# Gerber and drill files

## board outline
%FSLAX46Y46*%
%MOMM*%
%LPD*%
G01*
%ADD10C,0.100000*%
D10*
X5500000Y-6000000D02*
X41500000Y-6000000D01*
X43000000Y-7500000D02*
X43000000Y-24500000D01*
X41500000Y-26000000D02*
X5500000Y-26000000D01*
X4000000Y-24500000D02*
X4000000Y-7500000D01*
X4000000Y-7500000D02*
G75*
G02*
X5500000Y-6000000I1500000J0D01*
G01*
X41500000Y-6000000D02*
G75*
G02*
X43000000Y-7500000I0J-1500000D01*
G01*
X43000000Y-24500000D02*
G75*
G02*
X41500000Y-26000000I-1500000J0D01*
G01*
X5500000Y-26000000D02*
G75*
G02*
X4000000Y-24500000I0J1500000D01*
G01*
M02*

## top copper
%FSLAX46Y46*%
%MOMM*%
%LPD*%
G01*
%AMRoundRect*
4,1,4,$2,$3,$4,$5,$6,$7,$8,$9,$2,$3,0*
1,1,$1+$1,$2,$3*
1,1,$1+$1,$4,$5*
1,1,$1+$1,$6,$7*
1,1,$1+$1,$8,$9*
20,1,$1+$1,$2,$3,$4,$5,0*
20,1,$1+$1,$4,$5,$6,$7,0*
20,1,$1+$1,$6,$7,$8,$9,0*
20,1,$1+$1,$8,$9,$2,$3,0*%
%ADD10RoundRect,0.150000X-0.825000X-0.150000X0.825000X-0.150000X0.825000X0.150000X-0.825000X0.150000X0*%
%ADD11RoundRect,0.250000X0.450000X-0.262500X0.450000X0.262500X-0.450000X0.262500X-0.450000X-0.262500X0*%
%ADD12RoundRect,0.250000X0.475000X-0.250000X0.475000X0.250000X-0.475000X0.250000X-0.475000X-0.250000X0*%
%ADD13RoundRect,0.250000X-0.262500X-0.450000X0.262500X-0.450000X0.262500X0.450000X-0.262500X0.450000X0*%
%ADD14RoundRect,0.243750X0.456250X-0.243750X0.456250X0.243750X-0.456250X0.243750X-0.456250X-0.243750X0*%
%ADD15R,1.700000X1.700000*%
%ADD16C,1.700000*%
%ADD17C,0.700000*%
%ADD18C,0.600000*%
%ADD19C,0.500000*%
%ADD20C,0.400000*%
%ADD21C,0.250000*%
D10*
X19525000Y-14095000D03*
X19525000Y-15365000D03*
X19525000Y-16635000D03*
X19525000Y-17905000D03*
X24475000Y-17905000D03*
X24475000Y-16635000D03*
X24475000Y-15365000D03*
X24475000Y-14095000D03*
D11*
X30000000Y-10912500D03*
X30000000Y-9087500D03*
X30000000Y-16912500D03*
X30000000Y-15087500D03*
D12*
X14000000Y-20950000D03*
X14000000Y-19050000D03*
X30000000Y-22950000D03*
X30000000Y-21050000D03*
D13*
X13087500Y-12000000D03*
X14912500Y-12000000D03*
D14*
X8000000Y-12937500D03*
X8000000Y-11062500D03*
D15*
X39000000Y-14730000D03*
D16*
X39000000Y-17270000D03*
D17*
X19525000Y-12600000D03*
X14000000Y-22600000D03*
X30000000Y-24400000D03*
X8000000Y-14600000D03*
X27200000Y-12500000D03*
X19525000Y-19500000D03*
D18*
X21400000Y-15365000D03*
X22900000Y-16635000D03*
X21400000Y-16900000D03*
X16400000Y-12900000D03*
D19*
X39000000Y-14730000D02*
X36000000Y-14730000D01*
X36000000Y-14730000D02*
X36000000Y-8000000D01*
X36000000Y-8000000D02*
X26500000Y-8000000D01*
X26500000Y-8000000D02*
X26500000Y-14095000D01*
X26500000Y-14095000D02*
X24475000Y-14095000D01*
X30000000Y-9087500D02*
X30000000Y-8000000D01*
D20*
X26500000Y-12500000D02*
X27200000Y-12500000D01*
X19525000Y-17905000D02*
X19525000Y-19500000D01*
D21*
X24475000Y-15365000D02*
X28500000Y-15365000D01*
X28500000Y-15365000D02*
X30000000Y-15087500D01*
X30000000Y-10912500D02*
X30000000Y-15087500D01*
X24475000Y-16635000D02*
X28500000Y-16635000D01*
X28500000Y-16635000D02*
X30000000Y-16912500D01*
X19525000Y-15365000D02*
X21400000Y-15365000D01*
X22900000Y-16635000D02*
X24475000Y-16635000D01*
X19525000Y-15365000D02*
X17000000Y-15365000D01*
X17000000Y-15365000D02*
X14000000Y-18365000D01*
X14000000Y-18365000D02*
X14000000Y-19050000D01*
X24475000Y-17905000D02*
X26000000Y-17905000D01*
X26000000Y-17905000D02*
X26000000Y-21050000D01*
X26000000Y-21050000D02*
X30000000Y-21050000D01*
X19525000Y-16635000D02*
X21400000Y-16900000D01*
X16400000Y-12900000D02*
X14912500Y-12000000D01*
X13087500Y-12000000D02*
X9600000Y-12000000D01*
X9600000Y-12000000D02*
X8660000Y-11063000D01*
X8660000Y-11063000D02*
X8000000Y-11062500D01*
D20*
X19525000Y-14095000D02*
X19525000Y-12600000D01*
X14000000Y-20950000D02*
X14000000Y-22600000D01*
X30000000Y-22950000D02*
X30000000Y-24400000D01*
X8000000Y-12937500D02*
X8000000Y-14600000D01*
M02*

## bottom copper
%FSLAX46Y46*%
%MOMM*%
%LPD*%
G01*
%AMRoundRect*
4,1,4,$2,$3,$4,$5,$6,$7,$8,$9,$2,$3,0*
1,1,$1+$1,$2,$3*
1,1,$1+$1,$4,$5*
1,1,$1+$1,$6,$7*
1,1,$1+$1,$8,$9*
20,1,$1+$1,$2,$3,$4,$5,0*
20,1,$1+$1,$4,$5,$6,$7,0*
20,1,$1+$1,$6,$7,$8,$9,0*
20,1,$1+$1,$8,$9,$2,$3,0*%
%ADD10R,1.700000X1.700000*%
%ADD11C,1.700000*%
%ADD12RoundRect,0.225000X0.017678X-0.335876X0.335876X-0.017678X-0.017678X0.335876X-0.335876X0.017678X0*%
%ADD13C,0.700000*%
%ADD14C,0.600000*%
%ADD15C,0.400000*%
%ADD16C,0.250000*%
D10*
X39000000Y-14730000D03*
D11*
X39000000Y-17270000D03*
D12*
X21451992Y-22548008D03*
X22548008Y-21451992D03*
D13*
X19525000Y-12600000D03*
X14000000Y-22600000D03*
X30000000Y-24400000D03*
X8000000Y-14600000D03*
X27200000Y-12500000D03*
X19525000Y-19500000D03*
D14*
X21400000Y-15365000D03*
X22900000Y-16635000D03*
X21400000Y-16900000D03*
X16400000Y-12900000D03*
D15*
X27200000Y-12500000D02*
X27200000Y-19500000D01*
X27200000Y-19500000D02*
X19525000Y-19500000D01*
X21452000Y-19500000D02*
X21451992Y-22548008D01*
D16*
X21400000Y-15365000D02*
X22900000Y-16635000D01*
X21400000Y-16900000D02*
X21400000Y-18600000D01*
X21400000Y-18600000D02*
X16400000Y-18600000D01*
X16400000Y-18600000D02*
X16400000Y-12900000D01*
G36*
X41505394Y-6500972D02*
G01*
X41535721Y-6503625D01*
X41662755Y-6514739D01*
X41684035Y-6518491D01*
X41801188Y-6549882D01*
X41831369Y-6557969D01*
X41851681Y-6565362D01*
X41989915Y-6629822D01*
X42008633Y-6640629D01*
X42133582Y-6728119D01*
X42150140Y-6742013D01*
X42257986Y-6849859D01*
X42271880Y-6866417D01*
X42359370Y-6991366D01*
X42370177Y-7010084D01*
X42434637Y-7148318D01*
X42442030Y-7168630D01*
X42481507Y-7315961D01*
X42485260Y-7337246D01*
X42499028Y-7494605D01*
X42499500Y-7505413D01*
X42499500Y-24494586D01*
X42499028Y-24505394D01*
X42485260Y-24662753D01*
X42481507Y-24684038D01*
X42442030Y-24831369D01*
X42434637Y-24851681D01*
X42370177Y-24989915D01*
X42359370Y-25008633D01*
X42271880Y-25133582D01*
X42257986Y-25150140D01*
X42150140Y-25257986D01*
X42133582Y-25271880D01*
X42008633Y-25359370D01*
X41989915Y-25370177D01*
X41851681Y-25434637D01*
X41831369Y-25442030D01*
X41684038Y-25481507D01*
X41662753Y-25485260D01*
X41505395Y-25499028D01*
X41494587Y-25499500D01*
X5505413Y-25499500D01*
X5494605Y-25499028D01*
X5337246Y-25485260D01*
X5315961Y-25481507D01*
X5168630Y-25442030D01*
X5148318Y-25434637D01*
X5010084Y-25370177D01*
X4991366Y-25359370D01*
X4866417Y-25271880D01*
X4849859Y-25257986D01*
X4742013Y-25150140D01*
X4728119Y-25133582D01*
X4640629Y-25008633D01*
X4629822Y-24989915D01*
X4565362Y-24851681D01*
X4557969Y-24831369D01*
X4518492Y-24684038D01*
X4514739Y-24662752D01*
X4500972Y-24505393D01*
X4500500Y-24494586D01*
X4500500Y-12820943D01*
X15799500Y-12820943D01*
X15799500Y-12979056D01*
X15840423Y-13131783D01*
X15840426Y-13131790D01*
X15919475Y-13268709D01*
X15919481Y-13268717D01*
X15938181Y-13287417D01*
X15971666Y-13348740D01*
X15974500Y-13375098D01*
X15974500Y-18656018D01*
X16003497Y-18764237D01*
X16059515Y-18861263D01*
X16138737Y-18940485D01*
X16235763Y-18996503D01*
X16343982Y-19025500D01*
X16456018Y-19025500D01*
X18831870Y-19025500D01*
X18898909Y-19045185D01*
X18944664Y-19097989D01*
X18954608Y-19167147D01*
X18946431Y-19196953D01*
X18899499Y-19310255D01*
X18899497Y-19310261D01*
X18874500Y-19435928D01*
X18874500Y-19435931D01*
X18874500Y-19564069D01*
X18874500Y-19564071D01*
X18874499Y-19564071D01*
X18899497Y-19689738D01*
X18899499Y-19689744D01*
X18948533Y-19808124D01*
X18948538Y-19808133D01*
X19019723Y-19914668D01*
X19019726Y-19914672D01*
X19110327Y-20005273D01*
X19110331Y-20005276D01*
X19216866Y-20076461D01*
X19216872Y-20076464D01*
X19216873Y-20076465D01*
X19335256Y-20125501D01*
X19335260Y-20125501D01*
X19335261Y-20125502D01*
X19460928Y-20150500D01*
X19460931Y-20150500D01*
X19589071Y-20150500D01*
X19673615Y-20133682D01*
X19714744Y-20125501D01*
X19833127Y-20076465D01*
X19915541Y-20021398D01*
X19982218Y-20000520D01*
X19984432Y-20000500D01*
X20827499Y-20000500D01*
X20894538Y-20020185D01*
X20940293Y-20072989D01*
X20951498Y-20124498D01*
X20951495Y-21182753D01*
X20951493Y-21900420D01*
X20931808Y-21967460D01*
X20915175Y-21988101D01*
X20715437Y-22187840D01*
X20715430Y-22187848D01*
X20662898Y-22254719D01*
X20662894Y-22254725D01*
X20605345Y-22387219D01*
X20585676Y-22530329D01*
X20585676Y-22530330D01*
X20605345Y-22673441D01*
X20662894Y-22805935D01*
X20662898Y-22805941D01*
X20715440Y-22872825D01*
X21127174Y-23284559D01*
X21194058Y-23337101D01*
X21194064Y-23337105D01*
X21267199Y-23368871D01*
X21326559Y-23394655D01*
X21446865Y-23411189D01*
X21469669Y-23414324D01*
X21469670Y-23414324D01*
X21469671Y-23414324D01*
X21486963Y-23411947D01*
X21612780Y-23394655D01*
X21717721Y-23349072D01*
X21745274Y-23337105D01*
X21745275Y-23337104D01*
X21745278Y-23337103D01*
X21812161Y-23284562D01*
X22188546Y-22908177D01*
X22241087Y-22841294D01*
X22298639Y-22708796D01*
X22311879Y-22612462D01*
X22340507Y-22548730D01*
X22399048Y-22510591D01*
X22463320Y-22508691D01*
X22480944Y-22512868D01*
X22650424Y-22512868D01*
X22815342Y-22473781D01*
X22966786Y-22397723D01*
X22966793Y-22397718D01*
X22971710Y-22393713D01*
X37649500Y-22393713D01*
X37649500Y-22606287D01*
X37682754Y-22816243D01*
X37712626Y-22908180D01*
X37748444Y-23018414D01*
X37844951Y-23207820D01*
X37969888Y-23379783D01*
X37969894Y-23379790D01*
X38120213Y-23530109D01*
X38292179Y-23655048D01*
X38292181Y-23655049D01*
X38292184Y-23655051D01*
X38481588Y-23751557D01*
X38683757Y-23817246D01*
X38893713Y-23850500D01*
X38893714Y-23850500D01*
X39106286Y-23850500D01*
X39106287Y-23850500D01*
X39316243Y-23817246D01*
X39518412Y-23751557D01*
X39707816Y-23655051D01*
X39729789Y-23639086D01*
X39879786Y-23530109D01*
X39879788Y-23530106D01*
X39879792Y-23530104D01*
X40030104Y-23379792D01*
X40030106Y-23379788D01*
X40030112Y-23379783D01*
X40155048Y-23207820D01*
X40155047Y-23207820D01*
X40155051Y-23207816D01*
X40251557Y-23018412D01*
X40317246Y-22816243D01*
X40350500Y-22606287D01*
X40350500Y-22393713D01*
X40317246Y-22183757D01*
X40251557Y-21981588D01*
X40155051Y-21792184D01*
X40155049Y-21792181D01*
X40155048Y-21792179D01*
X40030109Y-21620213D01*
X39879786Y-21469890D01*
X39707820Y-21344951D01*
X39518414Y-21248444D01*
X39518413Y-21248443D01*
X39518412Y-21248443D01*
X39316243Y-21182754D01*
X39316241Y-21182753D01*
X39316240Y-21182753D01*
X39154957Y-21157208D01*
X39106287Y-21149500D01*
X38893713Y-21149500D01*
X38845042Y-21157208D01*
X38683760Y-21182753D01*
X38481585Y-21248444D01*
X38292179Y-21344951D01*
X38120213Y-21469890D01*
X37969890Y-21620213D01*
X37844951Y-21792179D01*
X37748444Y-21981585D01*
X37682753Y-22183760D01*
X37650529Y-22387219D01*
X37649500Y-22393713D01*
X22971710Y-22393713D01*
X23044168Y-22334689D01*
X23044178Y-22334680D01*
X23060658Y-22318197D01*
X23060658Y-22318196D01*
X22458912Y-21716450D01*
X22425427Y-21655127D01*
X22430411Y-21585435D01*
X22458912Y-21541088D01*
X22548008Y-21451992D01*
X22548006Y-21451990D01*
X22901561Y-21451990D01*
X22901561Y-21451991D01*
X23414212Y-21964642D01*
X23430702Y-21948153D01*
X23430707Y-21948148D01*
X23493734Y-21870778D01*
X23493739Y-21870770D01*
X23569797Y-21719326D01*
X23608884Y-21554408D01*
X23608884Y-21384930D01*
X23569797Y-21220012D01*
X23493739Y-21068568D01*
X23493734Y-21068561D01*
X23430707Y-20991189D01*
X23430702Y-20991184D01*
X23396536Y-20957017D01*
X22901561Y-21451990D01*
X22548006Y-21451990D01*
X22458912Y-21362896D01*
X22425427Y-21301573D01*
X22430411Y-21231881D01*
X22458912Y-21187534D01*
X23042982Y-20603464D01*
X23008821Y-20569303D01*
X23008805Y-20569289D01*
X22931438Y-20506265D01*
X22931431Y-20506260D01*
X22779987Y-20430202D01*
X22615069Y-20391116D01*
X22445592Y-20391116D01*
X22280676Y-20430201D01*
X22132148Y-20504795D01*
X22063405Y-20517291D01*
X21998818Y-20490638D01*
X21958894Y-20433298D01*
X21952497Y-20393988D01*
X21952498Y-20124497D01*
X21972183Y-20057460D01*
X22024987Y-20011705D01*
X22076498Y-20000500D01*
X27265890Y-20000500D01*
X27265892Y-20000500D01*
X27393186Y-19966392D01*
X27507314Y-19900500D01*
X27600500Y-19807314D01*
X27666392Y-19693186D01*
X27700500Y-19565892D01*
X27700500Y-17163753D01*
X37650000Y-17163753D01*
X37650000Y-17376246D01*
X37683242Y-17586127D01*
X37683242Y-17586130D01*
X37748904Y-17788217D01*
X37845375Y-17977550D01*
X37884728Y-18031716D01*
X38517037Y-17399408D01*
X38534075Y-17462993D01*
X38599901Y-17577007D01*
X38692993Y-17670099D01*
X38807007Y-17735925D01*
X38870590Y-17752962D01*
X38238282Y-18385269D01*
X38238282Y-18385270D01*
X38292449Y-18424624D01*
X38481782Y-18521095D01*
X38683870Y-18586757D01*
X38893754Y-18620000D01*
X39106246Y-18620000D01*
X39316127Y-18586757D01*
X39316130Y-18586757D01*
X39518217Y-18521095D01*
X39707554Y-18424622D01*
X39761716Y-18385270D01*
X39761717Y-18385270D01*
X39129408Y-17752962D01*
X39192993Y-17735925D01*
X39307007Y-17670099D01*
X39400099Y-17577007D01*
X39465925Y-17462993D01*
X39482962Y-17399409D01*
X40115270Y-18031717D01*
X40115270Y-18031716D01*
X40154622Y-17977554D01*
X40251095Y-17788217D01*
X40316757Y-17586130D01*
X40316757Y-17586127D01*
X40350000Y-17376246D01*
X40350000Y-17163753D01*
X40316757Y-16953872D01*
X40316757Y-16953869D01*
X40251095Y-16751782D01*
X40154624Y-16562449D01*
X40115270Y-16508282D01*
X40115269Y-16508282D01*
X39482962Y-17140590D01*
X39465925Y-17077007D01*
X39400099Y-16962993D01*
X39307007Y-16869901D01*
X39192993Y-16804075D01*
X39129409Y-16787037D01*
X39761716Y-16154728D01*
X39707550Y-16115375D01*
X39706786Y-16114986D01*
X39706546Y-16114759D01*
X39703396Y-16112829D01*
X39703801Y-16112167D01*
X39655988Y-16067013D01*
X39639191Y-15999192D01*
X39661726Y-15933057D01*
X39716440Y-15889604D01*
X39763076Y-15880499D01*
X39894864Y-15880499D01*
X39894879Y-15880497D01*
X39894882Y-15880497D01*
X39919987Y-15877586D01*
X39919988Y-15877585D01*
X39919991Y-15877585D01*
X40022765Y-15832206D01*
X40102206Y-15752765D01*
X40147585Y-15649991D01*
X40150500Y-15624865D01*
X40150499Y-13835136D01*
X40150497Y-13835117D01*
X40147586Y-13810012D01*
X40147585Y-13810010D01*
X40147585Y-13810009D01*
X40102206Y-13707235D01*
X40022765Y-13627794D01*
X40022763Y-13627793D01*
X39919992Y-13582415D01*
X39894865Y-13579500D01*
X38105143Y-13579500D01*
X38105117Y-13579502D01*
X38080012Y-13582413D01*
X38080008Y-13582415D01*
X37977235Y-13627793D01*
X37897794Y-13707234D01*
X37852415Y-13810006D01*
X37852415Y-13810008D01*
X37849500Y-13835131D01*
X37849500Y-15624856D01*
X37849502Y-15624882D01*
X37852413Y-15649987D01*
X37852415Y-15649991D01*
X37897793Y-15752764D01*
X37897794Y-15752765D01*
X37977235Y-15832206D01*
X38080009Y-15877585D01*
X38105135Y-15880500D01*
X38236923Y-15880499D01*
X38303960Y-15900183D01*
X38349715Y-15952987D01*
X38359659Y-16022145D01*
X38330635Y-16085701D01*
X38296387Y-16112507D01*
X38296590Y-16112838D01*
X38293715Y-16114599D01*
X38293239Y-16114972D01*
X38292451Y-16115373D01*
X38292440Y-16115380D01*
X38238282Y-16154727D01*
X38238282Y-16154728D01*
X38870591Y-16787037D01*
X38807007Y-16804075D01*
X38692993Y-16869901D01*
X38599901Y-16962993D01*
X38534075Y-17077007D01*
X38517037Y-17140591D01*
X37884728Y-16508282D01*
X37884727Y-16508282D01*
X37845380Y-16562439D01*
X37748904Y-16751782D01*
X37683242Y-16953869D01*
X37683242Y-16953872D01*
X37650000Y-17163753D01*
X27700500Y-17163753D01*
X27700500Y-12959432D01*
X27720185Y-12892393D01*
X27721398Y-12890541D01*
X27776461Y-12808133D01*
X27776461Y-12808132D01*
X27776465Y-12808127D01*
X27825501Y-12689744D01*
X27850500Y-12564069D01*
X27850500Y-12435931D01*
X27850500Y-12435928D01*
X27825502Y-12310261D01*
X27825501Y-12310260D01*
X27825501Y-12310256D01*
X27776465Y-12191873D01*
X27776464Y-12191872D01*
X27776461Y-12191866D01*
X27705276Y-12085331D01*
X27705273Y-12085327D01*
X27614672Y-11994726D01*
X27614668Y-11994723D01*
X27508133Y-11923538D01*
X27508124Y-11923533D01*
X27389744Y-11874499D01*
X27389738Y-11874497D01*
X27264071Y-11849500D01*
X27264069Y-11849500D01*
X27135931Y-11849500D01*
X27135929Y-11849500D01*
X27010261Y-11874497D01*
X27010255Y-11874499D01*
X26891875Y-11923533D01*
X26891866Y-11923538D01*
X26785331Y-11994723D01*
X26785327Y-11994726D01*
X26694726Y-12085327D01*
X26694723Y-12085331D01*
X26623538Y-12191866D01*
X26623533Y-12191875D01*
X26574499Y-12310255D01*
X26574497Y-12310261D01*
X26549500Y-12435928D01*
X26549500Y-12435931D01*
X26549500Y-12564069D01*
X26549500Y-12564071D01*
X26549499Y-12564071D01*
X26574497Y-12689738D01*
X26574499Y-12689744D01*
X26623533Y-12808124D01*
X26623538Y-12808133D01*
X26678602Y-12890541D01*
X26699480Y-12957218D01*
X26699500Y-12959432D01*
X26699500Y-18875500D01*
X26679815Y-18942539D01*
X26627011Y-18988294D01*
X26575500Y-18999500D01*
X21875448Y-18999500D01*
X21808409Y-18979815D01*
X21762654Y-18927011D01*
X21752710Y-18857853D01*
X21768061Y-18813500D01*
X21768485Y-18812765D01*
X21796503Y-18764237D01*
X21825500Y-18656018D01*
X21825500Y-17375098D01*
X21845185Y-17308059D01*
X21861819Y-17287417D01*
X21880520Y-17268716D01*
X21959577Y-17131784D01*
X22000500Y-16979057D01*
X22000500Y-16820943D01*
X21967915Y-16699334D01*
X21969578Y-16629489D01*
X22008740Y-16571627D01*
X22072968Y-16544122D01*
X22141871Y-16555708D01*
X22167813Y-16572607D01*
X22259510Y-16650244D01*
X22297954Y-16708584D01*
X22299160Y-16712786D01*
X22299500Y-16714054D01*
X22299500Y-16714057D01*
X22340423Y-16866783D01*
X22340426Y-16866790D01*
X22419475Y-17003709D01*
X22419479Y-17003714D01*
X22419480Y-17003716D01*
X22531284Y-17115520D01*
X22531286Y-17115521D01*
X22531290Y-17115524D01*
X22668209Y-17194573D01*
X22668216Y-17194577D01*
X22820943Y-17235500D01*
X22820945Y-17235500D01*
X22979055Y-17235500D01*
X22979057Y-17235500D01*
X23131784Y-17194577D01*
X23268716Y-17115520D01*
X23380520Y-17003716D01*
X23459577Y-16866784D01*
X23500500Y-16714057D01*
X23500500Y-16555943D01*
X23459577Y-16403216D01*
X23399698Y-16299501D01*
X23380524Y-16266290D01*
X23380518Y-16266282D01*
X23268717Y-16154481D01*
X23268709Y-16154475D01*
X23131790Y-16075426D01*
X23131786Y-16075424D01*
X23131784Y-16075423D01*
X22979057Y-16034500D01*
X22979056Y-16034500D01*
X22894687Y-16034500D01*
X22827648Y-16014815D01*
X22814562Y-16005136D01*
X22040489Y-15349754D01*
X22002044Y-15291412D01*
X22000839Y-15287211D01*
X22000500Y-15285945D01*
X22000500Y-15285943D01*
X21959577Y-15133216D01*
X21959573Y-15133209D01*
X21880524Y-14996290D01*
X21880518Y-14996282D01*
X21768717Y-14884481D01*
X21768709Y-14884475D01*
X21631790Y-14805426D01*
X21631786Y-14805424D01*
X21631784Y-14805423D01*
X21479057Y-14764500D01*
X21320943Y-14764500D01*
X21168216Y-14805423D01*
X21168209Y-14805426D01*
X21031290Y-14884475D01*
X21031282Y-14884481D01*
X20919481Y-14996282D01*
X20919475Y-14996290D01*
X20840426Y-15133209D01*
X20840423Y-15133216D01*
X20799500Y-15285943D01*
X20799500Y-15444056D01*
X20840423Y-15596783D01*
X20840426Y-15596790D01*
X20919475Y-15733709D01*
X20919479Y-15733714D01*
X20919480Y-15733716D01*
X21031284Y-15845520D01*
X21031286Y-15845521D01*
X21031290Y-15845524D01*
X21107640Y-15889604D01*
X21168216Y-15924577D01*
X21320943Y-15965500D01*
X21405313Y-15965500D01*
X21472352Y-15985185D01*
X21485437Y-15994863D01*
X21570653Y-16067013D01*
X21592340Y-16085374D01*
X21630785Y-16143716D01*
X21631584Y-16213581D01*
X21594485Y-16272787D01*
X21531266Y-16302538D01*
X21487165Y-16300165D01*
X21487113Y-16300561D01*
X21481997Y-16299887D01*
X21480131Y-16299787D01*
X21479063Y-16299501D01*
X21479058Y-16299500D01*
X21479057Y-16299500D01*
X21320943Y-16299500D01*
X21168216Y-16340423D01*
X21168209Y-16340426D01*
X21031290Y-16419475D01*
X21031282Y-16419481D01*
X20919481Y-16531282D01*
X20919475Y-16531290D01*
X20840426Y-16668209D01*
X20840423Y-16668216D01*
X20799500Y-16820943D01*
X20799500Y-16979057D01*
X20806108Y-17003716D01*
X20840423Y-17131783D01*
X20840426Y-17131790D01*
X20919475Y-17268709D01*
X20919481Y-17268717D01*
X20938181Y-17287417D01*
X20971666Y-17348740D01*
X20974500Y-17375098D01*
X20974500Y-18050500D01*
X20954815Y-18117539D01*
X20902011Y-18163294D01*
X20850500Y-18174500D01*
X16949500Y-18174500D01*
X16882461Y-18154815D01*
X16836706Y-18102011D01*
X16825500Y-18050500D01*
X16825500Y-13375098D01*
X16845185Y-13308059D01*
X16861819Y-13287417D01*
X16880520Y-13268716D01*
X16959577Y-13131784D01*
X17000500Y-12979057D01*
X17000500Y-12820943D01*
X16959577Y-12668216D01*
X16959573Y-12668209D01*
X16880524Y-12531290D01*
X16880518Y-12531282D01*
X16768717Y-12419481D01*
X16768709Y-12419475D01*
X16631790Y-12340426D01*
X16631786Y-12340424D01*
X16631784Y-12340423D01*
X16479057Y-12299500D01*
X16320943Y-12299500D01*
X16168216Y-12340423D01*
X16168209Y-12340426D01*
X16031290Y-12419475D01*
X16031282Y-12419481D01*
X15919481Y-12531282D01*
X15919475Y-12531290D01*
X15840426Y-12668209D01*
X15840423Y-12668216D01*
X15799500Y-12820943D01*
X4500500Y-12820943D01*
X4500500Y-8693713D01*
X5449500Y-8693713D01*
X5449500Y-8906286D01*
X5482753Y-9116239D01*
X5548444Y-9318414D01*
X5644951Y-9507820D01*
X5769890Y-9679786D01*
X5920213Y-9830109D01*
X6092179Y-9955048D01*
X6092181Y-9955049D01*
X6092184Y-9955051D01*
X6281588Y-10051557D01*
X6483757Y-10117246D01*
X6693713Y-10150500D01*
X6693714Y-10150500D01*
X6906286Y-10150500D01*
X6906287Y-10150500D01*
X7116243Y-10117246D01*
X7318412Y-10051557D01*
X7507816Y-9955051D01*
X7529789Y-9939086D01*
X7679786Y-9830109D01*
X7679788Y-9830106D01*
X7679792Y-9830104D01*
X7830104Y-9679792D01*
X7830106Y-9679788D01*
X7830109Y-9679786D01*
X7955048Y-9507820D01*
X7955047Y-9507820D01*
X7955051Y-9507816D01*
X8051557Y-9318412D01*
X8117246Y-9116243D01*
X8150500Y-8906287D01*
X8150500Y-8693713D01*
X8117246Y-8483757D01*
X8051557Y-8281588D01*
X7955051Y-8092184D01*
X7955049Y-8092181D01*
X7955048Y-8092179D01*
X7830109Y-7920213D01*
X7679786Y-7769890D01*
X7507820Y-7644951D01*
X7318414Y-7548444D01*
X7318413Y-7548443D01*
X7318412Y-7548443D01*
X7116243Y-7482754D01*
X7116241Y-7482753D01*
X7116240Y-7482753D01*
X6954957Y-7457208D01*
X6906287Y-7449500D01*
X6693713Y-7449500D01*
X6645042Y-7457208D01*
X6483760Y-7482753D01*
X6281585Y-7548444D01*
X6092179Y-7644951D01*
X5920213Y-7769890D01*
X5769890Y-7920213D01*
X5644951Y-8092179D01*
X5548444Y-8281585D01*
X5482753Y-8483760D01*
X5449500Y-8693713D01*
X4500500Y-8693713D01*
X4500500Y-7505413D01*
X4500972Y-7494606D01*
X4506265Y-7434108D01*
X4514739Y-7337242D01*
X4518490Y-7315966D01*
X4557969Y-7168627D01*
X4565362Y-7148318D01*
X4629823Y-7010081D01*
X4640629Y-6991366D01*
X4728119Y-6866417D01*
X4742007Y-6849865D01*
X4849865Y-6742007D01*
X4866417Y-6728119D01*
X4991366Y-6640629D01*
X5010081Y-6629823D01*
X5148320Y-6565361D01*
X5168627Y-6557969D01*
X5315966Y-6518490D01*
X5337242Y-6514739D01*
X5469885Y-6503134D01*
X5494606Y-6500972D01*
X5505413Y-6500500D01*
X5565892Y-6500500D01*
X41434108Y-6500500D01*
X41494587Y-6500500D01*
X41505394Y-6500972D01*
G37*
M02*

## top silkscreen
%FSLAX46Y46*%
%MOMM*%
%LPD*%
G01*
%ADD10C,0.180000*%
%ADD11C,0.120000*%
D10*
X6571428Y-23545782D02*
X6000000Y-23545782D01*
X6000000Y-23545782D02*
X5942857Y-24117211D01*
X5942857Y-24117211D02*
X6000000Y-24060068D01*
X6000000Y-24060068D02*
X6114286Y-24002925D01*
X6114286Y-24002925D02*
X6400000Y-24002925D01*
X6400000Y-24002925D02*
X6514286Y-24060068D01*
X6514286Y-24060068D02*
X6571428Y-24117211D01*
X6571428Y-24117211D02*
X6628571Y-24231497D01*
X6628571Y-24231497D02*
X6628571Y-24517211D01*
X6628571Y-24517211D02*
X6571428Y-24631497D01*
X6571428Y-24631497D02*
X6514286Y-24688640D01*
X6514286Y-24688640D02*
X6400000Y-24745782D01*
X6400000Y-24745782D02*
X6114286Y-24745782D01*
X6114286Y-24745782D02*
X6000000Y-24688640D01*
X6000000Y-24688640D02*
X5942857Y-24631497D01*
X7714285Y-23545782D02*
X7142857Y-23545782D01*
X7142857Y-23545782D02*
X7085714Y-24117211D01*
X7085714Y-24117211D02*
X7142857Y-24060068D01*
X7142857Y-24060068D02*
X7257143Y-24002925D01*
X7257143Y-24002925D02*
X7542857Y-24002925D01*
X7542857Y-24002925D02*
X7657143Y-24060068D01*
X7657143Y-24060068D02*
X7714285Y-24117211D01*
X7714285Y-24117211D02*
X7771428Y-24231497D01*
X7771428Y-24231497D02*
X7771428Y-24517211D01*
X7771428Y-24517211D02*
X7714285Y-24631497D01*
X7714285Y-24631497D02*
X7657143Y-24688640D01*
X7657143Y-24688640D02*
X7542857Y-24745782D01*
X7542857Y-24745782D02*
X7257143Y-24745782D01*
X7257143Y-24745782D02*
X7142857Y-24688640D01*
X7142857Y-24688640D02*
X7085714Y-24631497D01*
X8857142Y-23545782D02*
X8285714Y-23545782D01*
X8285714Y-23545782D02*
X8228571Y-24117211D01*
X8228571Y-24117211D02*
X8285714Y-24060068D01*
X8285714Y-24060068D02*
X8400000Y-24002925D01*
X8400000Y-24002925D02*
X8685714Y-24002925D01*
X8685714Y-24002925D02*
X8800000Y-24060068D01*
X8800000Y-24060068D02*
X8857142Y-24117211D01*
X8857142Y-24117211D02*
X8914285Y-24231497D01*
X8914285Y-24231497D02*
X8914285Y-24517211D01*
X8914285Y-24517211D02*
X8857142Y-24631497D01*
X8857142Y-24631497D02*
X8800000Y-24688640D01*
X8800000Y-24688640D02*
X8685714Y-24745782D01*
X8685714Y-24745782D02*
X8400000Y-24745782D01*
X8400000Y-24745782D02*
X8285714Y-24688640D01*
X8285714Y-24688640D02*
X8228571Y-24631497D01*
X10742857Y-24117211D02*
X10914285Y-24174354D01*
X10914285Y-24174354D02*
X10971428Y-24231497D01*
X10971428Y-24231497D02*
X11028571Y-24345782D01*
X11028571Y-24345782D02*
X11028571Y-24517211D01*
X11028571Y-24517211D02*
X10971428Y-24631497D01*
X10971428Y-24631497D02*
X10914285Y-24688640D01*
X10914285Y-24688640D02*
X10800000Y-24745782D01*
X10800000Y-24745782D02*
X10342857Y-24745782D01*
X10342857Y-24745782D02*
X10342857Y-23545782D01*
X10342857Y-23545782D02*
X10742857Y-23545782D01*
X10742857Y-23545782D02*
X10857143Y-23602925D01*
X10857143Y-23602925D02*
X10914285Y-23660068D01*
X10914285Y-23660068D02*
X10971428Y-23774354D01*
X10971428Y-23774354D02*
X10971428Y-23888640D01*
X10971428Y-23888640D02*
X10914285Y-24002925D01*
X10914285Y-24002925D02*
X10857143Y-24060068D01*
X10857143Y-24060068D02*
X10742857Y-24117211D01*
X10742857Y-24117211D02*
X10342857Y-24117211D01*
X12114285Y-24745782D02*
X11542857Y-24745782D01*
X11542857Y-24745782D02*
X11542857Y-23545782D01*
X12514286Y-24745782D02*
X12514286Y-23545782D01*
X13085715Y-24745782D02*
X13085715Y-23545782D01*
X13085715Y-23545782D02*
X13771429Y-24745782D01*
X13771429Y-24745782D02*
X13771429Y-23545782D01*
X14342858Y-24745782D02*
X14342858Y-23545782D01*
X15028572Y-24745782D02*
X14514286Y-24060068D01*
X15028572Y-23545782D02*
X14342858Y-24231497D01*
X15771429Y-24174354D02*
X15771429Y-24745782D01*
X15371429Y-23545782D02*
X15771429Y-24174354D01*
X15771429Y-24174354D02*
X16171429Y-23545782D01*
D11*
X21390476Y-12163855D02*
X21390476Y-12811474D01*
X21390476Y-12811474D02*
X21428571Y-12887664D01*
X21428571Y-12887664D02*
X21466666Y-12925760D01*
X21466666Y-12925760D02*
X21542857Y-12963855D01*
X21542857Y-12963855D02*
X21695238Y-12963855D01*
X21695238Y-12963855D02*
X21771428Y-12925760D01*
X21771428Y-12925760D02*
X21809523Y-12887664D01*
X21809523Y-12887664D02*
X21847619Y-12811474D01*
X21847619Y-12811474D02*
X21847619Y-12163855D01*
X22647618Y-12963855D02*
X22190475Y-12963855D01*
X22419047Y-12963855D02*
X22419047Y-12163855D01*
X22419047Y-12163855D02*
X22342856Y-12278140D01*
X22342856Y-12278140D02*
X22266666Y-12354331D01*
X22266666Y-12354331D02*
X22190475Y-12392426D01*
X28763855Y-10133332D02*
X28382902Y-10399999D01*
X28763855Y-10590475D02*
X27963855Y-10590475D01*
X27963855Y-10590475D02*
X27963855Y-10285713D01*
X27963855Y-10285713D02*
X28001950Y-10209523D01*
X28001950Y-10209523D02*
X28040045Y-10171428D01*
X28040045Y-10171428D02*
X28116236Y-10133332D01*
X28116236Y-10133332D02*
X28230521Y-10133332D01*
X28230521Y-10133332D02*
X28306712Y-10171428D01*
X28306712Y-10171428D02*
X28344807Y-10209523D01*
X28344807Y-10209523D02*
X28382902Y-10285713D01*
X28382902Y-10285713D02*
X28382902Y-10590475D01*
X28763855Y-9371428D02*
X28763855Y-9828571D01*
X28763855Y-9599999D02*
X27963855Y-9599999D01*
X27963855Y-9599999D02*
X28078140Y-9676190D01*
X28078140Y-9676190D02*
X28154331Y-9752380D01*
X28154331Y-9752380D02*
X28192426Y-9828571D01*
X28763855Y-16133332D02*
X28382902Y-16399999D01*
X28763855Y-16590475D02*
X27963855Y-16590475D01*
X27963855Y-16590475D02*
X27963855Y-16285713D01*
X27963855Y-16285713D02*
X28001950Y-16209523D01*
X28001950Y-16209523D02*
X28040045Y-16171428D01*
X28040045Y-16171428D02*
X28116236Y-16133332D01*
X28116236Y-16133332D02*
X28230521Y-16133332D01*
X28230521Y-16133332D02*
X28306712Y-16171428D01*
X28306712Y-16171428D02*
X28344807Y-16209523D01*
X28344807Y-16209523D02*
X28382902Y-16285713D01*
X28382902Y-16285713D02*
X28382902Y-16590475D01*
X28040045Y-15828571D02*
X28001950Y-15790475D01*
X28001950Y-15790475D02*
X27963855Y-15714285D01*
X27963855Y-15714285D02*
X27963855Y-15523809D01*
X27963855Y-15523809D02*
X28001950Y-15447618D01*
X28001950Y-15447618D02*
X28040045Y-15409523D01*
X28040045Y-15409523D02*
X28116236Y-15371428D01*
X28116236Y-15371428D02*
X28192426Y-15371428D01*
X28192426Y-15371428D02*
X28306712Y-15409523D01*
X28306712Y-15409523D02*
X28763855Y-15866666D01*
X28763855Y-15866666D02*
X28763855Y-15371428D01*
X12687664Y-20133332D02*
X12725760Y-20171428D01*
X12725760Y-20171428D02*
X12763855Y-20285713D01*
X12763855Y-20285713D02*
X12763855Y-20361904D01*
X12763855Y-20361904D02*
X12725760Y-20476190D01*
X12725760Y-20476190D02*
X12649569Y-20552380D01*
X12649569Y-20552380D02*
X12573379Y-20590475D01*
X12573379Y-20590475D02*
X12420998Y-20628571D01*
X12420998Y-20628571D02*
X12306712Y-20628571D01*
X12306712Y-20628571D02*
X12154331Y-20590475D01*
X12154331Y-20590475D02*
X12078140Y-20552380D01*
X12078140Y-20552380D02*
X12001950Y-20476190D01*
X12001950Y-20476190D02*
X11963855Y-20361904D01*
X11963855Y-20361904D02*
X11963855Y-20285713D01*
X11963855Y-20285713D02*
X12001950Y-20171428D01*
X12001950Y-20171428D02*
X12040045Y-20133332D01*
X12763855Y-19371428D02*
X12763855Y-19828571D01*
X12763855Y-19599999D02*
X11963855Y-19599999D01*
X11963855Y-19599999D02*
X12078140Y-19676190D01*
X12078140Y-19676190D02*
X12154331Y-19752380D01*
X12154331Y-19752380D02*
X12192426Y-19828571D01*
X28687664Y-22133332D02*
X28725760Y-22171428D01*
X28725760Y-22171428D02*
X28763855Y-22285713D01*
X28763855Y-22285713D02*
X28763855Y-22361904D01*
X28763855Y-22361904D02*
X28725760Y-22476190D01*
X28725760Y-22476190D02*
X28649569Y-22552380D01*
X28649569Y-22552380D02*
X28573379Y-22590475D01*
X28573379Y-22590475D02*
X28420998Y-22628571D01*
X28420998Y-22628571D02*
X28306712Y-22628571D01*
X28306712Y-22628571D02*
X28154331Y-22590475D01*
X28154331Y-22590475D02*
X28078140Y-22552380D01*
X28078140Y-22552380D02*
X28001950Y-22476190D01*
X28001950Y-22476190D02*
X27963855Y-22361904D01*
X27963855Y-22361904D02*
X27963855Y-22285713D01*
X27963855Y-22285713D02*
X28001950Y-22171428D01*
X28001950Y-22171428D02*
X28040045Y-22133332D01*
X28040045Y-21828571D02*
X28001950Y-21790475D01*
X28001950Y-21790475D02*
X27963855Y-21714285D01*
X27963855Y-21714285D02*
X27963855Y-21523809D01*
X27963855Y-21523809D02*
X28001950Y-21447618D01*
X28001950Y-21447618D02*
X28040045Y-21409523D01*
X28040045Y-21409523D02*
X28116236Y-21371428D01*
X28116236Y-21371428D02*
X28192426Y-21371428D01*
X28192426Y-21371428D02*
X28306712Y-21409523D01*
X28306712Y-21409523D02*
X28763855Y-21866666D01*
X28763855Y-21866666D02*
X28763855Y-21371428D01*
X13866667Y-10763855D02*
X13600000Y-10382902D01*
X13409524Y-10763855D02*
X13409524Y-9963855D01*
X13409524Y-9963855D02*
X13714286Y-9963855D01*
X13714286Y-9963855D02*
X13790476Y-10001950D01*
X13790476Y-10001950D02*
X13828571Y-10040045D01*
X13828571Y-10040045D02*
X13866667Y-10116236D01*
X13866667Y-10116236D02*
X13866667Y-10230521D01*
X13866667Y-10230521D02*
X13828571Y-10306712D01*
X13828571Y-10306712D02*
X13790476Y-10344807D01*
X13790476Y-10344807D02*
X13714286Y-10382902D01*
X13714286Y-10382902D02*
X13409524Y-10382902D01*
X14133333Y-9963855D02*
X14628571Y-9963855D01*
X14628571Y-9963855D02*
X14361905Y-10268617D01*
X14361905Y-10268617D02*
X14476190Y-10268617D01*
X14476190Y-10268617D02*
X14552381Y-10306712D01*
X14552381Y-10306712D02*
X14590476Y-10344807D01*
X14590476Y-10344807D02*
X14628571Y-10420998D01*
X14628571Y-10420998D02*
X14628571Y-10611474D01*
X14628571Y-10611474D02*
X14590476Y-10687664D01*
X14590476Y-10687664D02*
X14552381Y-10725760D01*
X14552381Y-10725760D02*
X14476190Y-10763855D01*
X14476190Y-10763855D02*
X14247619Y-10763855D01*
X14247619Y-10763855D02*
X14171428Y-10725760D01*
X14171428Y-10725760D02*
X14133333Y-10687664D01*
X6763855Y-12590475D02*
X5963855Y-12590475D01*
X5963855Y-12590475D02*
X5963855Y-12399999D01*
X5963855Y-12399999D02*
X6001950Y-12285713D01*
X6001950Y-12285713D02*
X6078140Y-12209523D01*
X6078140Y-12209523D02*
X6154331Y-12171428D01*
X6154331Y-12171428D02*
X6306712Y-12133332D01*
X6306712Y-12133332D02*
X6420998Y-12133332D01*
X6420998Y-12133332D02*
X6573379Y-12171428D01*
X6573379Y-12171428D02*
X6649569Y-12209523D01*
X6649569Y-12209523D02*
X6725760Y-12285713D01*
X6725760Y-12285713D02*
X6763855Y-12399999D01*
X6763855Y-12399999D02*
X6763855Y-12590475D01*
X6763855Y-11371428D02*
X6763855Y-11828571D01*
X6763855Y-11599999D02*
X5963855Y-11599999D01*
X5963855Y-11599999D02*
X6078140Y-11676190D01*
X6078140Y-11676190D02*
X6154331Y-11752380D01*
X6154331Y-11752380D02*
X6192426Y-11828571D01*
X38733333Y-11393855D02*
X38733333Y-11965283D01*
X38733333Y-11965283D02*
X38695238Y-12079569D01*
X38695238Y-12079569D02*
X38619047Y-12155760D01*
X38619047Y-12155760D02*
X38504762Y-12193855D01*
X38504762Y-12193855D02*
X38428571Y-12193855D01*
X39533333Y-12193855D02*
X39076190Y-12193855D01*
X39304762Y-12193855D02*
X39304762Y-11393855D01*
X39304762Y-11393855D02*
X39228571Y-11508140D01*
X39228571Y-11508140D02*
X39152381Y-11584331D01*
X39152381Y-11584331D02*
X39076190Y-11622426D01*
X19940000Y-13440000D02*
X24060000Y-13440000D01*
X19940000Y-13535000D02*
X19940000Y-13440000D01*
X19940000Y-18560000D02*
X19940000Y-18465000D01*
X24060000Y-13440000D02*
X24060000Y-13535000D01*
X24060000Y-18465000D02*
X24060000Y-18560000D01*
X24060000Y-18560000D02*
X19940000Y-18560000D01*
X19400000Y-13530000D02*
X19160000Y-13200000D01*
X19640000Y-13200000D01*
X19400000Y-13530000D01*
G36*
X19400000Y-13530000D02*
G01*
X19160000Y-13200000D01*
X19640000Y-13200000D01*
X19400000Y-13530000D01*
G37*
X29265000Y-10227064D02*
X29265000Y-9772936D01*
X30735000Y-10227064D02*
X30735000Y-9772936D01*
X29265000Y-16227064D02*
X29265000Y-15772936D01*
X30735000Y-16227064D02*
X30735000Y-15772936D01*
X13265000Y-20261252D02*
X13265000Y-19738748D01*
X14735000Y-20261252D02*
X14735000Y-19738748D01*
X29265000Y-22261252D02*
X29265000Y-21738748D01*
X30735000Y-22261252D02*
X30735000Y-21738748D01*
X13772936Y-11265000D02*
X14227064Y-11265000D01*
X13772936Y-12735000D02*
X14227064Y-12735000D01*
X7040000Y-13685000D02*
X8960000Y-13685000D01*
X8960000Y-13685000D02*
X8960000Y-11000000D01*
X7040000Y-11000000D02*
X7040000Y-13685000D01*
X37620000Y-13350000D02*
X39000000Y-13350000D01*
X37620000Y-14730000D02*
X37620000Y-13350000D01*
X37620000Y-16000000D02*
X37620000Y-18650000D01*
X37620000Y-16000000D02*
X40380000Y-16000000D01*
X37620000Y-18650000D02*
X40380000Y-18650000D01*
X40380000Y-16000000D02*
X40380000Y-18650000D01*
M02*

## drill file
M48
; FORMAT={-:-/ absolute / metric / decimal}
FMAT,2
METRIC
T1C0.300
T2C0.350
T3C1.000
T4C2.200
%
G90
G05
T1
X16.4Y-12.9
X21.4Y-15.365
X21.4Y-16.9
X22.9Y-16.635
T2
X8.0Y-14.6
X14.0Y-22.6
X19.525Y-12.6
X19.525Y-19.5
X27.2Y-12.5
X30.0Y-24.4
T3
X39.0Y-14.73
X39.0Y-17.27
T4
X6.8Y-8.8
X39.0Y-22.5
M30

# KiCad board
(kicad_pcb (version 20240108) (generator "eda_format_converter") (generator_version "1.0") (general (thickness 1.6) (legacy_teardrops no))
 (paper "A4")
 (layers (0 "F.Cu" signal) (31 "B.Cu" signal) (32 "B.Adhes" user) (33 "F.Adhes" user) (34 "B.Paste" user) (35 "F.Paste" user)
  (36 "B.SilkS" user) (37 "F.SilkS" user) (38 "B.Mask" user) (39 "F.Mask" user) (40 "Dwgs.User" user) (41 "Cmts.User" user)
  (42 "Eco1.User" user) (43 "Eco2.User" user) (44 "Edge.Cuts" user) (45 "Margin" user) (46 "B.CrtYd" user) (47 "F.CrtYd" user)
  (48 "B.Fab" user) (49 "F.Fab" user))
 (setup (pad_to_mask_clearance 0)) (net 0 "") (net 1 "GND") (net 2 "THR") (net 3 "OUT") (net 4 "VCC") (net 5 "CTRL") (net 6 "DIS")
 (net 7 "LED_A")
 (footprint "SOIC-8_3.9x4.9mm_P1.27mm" (layer "F.Cu") (at 22 16)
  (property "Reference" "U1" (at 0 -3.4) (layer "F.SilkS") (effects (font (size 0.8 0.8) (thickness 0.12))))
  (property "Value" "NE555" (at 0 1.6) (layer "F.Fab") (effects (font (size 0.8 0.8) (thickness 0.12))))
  (fp_line (start -2.06 -2.56) (end 2.06 -2.56) (stroke (width 0.12) (type solid)) (layer "F.SilkS"))
  (fp_line (start -2.06 -2.465) (end -2.06 -2.56) (stroke (width 0.12) (type solid)) (layer "F.SilkS"))
  (fp_line (start -2.06 2.56) (end -2.06 2.465) (stroke (width 0.12) (type solid)) (layer "F.SilkS"))
  (fp_line (start 2.06 -2.56) (end 2.06 -2.465) (stroke (width 0.12) (type solid)) (layer "F.SilkS"))
  (fp_line (start 2.06 2.465) (end 2.06 2.56) (stroke (width 0.12) (type solid)) (layer "F.SilkS"))
  (fp_line (start 2.06 2.56) (end -2.06 2.56) (stroke (width 0.12) (type solid)) (layer "F.SilkS"))
  (fp_poly (pts (xy -2.6 -2.47) (xy -2.84 -2.8) (xy -2.36 -2.8)) (stroke (width 0.12) (type solid)) (fill solid) (layer "F.SilkS"))
  (pad "1" smd roundrect (at -2.475 -1.905) (size 1.95 0.6) (layers "F.Cu" "F.Paste" "F.Mask") (roundrect_rratio 0.25) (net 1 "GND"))
  (pad "2" smd roundrect (at -2.475 -0.635) (size 1.95 0.6) (layers "F.Cu" "F.Paste" "F.Mask") (roundrect_rratio 0.25) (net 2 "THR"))
  (pad "3" smd roundrect (at -2.475 0.635) (size 1.95 0.6) (layers "F.Cu" "F.Paste" "F.Mask") (roundrect_rratio 0.25) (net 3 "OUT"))
  (pad "4" smd roundrect (at -2.475 1.905) (size 1.95 0.6) (layers "F.Cu" "F.Paste" "F.Mask") (roundrect_rratio 0.25) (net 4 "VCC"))
  (pad "5" smd roundrect (at 2.475 1.905) (size 1.95 0.6) (layers "F.Cu" "F.Paste" "F.Mask") (roundrect_rratio 0.25) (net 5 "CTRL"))
  (pad "6" smd roundrect (at 2.475 0.635) (size 1.95 0.6) (layers "F.Cu" "F.Paste" "F.Mask") (roundrect_rratio 0.25) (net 2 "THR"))
  (pad "7" smd roundrect (at 2.475 -0.635) (size 1.95 0.6) (layers "F.Cu" "F.Paste" "F.Mask") (roundrect_rratio 0.25) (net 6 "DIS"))
  (pad "8" smd roundrect (at 2.475 -1.905) (size 1.95 0.6) (layers "F.Cu" "F.Paste" "F.Mask") (roundrect_rratio 0.25) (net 4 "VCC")))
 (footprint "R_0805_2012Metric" (layer "F.Cu") (at 30 10 90)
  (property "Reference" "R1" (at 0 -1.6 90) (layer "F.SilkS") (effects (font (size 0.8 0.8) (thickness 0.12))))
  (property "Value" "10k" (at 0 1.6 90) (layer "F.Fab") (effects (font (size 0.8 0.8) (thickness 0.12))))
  (fp_line (start -0.227064 -0.735) (end 0.227064 -0.735) (stroke (width 0.12) (type solid)) (layer "F.SilkS"))
  (fp_line (start -0.227064 0.735) (end 0.227064 0.735) (stroke (width 0.12) (type solid)) (layer "F.SilkS"))
  (pad "1" smd roundrect (at -0.9125 0 90) (size 1.025 1.4) (layers "F.Cu" "F.Paste" "F.Mask") (roundrect_rratio 0.243902) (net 6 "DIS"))
  (pad "2" smd roundrect (at 0.9125 0 90) (size 1.025 1.4) (layers "F.Cu" "F.Paste" "F.Mask") (roundrect_rratio 0.243902) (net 4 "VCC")))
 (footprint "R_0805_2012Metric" (layer "F.Cu") (at 30 16 90)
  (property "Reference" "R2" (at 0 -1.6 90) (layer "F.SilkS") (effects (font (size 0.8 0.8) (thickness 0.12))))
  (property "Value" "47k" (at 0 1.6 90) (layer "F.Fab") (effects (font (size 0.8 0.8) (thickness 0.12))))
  (fp_line (start -0.227064 -0.735) (end 0.227064 -0.735) (stroke (width 0.12) (type solid)) (layer "F.SilkS"))
  (fp_line (start -0.227064 0.735) (end 0.227064 0.735) (stroke (width 0.12) (type solid)) (layer "F.SilkS"))
  (pad "1" smd roundrect (at -0.9125 0 90) (size 1.025 1.4) (layers "F.Cu" "F.Paste" "F.Mask") (roundrect_rratio 0.243902) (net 2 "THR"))
  (pad "2" smd roundrect (at 0.9125 0 90) (size 1.025 1.4) (layers "F.Cu" "F.Paste" "F.Mask") (roundrect_rratio 0.243902) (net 6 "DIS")))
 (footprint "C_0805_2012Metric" (layer "F.Cu") (at 14 20 90)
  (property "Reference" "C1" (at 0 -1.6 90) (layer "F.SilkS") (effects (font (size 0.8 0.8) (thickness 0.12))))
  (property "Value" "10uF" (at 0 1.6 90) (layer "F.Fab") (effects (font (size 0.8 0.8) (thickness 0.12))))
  (fp_line (start -0.261252 -0.735) (end 0.261252 -0.735) (stroke (width 0.12) (type solid)) (layer "F.SilkS"))
  (fp_line (start -0.261252 0.735) (end 0.261252 0.735) (stroke (width 0.12) (type solid)) (layer "F.SilkS"))
  (pad "1" smd roundrect (at -0.95 0 90) (size 1 1.45) (layers "F.Cu" "F.Paste" "F.Mask") (roundrect_rratio 0.25) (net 1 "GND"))
  (pad "2" smd roundrect (at 0.95 0 90) (size 1 1.45) (layers "F.Cu" "F.Paste" "F.Mask") (roundrect_rratio 0.25) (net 2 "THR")))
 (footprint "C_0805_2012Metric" (layer "F.Cu") (at 30 22 90)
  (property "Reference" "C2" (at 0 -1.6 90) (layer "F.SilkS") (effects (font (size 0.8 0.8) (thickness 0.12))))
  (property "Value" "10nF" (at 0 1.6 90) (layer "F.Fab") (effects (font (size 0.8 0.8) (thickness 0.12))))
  (fp_line (start -0.261252 -0.735) (end 0.261252 -0.735) (stroke (width 0.12) (type solid)) (layer "F.SilkS"))
  (fp_line (start -0.261252 0.735) (end 0.261252 0.735) (stroke (width 0.12) (type solid)) (layer "F.SilkS"))
  (pad "1" smd roundrect (at -0.95 0 90) (size 1 1.45) (layers "F.Cu" "F.Paste" "F.Mask") (roundrect_rratio 0.25) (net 1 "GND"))
  (pad "2" smd roundrect (at 0.95 0 90) (size 1 1.45) (layers "F.Cu" "F.Paste" "F.Mask") (roundrect_rratio 0.25) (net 5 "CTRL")))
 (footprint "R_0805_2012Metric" (layer "F.Cu") (at 14 12)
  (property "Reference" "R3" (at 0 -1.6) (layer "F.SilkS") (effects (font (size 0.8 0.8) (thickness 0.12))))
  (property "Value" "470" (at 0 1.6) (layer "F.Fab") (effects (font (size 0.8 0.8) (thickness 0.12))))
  (fp_line (start -0.227064 -0.735) (end 0.227064 -0.735) (stroke (width 0.12) (type solid)) (layer "F.SilkS"))
  (fp_line (start -0.227064 0.735) (end 0.227064 0.735) (stroke (width 0.12) (type solid)) (layer "F.SilkS"))
  (pad "1" smd roundrect (at -0.9125 0) (size 1.025 1.4) (layers "F.Cu" "F.Paste" "F.Mask") (roundrect_rratio 0.243902) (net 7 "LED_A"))
  (pad "2" smd roundrect (at 0.9125 0) (size 1.025 1.4) (layers "F.Cu" "F.Paste" "F.Mask") (roundrect_rratio 0.243902) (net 3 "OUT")))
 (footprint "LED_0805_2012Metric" (layer "F.Cu") (at 8 12 90)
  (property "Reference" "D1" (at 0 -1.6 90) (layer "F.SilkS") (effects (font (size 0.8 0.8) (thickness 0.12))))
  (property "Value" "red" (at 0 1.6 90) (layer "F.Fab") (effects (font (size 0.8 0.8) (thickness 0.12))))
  (fp_line (start -1.685 -0.96) (end -1.685 0.96) (stroke (width 0.12) (type solid)) (layer "F.SilkS"))
  (fp_line (start -1.685 0.96) (end 1 0.96) (stroke (width 0.12) (type solid)) (layer "F.SilkS"))
  (fp_line (start 1 -0.96) (end -1.685 -0.96) (stroke (width 0.12) (type solid)) (layer "F.SilkS"))
  (pad "1" smd roundrect (at -0.9375 0 90) (size 0.975 1.4) (layers "F.Cu" "F.Paste" "F.Mask") (roundrect_rratio 0.25) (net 1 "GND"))
  (pad "2" smd roundrect (at 0.9375 0 90) (size 0.975 1.4) (layers "F.Cu" "F.Paste" "F.Mask") (roundrect_rratio 0.25) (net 7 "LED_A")))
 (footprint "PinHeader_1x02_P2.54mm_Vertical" (layer "F.Cu") (at 39 14.73)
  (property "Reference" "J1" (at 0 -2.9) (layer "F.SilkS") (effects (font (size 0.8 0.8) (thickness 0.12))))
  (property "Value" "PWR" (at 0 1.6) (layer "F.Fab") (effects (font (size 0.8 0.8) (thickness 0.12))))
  (fp_line (start -1.38 -1.38) (end 0 -1.38) (stroke (width 0.12) (type solid)) (layer "F.SilkS"))
  (fp_line (start -1.38 0) (end -1.38 -1.38) (stroke (width 0.12) (type solid)) (layer "F.SilkS"))
  (fp_line (start -1.38 1.27) (end -1.38 3.92) (stroke (width 0.12) (type solid)) (layer "F.SilkS"))
  (fp_line (start -1.38 1.27) (end 1.38 1.27) (stroke (width 0.12) (type solid)) (layer "F.SilkS"))
  (fp_line (start -1.38 3.92) (end 1.38 3.92) (stroke (width 0.12) (type solid)) (layer "F.SilkS"))
  (fp_line (start 1.38 1.27) (end 1.38 3.92) (stroke (width 0.12) (type solid)) (layer "F.SilkS"))
  (pad "1" thru_hole rect (at 0 0) (size 1.7 1.7) (drill 1) (layers "*.Cu" "*.Mask") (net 4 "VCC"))
  (pad "2" thru_hole circle (at 0 2.54) (size 1.7 1.7) (drill 1) (layers "*.Cu" "*.Mask") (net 1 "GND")))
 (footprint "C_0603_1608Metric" (layer "B.Cu") (at 22 22 45)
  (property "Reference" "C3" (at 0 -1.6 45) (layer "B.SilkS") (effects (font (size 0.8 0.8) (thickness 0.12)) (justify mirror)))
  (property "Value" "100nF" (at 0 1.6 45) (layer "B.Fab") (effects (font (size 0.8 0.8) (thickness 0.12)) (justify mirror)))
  (pad "1" smd roundrect (at -0.775 0 45) (size 0.9 0.95) (layers "B.Cu" "B.Paste" "B.Mask") (roundrect_rratio 0.25) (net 4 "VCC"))
  (pad "2" smd roundrect (at 0.775 0 45) (size 0.9 0.95) (layers "B.Cu" "B.Paste" "B.Mask") (roundrect_rratio 0.25) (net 1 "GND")))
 (gr_line (start 5.5 6) (end 41.5 6) (stroke (width 0.1) (type solid)) (layer "Edge.Cuts"))
 (gr_line (start 43 7.5) (end 43 24.5) (stroke (width 0.1) (type solid)) (layer "Edge.Cuts"))
 (gr_line (start 41.5 26) (end 5.5 26) (stroke (width 0.1) (type solid)) (layer "Edge.Cuts"))
 (gr_line (start 4 24.5) (end 4 7.5) (stroke (width 0.1) (type solid)) (layer "Edge.Cuts"))
 (gr_arc (start 4 7.5) (mid 4.43934 6.43934) (end 5.5 6) (stroke (width 0.1) (type solid)) (layer "Edge.Cuts"))
 (gr_arc (start 41.5 6) (mid 42.56066 6.43934) (end 43 7.5) (stroke (width 0.1) (type solid)) (layer "Edge.Cuts"))
 (gr_arc (start 43 24.5) (mid 42.56066 25.56066) (end 41.5 26) (stroke (width 0.1) (type solid)) (layer "Edge.Cuts"))
 (gr_arc (start 5.5 26) (mid 4.43934 25.56066) (end 4 24.5) (stroke (width 0.1) (type solid)) (layer "Edge.Cuts"))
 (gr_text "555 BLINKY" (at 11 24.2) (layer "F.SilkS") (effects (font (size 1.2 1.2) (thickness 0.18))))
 (segment (start 39 14.73) (end 36 14.73) (width 0.5) (layer "F.Cu") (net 4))
 (segment (start 36 14.73) (end 36 8) (width 0.5) (layer "F.Cu") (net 4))
 (segment (start 36 8) (end 26.5 8) (width 0.5) (layer "F.Cu") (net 4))
 (segment (start 26.5 8) (end 26.5 14.095) (width 0.5) (layer "F.Cu") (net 4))
 (segment (start 26.5 14.095) (end 24.475 14.095) (width 0.5) (layer "F.Cu") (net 4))
 (segment (start 30 9.0875) (end 30 8) (width 0.5) (layer "F.Cu") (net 4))
 (segment (start 26.5 12.5) (end 27.2 12.5) (width 0.4) (layer "F.Cu") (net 4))
 (segment (start 27.2 12.5) (end 27.2 19.5) (width 0.4) (layer "B.Cu") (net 4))
 (segment (start 27.2 19.5) (end 19.525 19.5) (width 0.4) (layer "B.Cu") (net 4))
 (segment (start 21.452 19.5) (end 21.451992 22.548008) (width 0.4) (layer "B.Cu") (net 4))
 (segment (start 19.525 17.905) (end 19.525 19.5) (width 0.4) (layer "F.Cu") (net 4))
 (segment (start 24.475 15.365) (end 28.5 15.365) (width 0.25) (layer "F.Cu") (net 6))
 (segment (start 28.5 15.365) (end 30 15.0875) (width 0.25) (layer "F.Cu") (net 6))
 (segment (start 30 10.9125) (end 30 15.0875) (width 0.25) (layer "F.Cu") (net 6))
 (segment (start 24.475 16.635) (end 28.5 16.635) (width 0.25) (layer "F.Cu") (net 2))
 (segment (start 28.5 16.635) (end 30 16.9125) (width 0.25) (layer "F.Cu") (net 2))
 (segment (start 19.525 15.365) (end 21.4 15.365) (width 0.25) (layer "F.Cu") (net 2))
 (segment (start 21.4 15.365) (end 22.9 16.635) (width 0.25) (layer "B.Cu") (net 2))
 (segment (start 22.9 16.635) (end 24.475 16.635) (width 0.25) (layer "F.Cu") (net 2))
 (segment (start 19.525 15.365) (end 17 15.365) (width 0.25) (layer "F.Cu") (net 2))
 (segment (start 17 15.365) (end 14 18.365) (width 0.25) (layer "F.Cu") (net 2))
 (segment (start 14 18.365) (end 14 19.05) (width 0.25) (layer "F.Cu") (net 2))
 (segment (start 24.475 17.905) (end 26 17.905) (width 0.25) (layer "F.Cu") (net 5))
 (segment (start 26 17.905) (end 26 21.05) (width 0.25) (layer "F.Cu") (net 5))
 (segment (start 26 21.05) (end 30 21.05) (width 0.25) (layer "F.Cu") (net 5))
 (segment (start 19.525 16.635) (end 21.4 16.9) (width 0.25) (layer "F.Cu") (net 3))
 (segment (start 21.4 16.9) (end 21.4 18.6) (width 0.25) (layer "B.Cu") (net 3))
 (segment (start 21.4 18.6) (end 16.4 18.6) (width 0.25) (layer "B.Cu") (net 3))
 (segment (start 16.4 18.6) (end 16.4 12.9) (width 0.25) (layer "B.Cu") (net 3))
 (segment (start 16.4 12.9) (end 14.9125 12) (width 0.25) (layer "F.Cu") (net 3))
 (segment (start 13.0875 12) (end 9.6 12) (width 0.25) (layer "F.Cu") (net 7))
 (segment (start 9.6 12) (end 8.66 11.063) (width 0.25) (layer "F.Cu") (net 7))
 (segment (start 8.66 11.063) (end 8 11.0625) (width 0.25) (layer "F.Cu") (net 7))
 (segment (start 19.525 14.095) (end 19.525 12.6) (width 0.4) (layer "F.Cu") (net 1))
 (segment (start 14 20.95) (end 14 22.6) (width 0.4) (layer "F.Cu") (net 1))
 (segment (start 30 22.95) (end 30 24.4) (width 0.4) (layer "F.Cu") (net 1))
 (segment (start 8 12.9375) (end 8 14.6) (width 0.4) (layer "F.Cu") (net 1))
 (via (at 19.525 12.6) (size 0.7) (drill 0.35) (layers "F.Cu" "B.Cu") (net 1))
 (via (at 14 22.6) (size 0.7) (drill 0.35) (layers "F.Cu" "B.Cu") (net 1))
 (via (at 30 24.4) (size 0.7) (drill 0.35) (layers "F.Cu" "B.Cu") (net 1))
 (via (at 8 14.6) (size 0.7) (drill 0.35) (layers "F.Cu" "B.Cu") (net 1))
 (via (at 27.2 12.5) (size 0.7) (drill 0.35) (layers "F.Cu" "B.Cu") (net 4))
 (via (at 19.525 19.5) (size 0.7) (drill 0.35) (layers "F.Cu" "B.Cu") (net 4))
 (via (at 21.4 15.365) (size 0.6) (drill 0.3) (layers "F.Cu" "B.Cu") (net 2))
 (via (at 22.9 16.635) (size 0.6) (drill 0.3) (layers "F.Cu" "B.Cu") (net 2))
 (via (at 21.4 16.9) (size 0.6) (drill 0.3) (layers "F.Cu" "B.Cu") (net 3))
 (via (at 16.4 12.9) (size 0.6) (drill 0.3) (layers "F.Cu" "B.Cu") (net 3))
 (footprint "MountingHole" (layer "F.Cu") (at 6.8 8.8)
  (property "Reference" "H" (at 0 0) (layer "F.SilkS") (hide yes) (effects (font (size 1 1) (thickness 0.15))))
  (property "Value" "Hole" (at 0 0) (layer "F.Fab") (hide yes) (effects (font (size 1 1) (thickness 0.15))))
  (pad "" np_thru_hole circle (at 0 0) (size 2.2 2.2) (drill 2.2) (layers "*.Cu" "*.Mask")))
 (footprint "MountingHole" (layer "F.Cu") (at 39 22.5)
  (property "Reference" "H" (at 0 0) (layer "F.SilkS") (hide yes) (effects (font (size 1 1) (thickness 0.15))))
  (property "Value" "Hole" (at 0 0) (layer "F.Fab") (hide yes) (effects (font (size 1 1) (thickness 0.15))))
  (pad "" np_thru_hole circle (at 0 0) (size 2.2 2.2) (drill 2.2) (layers "*.Cu" "*.Mask")))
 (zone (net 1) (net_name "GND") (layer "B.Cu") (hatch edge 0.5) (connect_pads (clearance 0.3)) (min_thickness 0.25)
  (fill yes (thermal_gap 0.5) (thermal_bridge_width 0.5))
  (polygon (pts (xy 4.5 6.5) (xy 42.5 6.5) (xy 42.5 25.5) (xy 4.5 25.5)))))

